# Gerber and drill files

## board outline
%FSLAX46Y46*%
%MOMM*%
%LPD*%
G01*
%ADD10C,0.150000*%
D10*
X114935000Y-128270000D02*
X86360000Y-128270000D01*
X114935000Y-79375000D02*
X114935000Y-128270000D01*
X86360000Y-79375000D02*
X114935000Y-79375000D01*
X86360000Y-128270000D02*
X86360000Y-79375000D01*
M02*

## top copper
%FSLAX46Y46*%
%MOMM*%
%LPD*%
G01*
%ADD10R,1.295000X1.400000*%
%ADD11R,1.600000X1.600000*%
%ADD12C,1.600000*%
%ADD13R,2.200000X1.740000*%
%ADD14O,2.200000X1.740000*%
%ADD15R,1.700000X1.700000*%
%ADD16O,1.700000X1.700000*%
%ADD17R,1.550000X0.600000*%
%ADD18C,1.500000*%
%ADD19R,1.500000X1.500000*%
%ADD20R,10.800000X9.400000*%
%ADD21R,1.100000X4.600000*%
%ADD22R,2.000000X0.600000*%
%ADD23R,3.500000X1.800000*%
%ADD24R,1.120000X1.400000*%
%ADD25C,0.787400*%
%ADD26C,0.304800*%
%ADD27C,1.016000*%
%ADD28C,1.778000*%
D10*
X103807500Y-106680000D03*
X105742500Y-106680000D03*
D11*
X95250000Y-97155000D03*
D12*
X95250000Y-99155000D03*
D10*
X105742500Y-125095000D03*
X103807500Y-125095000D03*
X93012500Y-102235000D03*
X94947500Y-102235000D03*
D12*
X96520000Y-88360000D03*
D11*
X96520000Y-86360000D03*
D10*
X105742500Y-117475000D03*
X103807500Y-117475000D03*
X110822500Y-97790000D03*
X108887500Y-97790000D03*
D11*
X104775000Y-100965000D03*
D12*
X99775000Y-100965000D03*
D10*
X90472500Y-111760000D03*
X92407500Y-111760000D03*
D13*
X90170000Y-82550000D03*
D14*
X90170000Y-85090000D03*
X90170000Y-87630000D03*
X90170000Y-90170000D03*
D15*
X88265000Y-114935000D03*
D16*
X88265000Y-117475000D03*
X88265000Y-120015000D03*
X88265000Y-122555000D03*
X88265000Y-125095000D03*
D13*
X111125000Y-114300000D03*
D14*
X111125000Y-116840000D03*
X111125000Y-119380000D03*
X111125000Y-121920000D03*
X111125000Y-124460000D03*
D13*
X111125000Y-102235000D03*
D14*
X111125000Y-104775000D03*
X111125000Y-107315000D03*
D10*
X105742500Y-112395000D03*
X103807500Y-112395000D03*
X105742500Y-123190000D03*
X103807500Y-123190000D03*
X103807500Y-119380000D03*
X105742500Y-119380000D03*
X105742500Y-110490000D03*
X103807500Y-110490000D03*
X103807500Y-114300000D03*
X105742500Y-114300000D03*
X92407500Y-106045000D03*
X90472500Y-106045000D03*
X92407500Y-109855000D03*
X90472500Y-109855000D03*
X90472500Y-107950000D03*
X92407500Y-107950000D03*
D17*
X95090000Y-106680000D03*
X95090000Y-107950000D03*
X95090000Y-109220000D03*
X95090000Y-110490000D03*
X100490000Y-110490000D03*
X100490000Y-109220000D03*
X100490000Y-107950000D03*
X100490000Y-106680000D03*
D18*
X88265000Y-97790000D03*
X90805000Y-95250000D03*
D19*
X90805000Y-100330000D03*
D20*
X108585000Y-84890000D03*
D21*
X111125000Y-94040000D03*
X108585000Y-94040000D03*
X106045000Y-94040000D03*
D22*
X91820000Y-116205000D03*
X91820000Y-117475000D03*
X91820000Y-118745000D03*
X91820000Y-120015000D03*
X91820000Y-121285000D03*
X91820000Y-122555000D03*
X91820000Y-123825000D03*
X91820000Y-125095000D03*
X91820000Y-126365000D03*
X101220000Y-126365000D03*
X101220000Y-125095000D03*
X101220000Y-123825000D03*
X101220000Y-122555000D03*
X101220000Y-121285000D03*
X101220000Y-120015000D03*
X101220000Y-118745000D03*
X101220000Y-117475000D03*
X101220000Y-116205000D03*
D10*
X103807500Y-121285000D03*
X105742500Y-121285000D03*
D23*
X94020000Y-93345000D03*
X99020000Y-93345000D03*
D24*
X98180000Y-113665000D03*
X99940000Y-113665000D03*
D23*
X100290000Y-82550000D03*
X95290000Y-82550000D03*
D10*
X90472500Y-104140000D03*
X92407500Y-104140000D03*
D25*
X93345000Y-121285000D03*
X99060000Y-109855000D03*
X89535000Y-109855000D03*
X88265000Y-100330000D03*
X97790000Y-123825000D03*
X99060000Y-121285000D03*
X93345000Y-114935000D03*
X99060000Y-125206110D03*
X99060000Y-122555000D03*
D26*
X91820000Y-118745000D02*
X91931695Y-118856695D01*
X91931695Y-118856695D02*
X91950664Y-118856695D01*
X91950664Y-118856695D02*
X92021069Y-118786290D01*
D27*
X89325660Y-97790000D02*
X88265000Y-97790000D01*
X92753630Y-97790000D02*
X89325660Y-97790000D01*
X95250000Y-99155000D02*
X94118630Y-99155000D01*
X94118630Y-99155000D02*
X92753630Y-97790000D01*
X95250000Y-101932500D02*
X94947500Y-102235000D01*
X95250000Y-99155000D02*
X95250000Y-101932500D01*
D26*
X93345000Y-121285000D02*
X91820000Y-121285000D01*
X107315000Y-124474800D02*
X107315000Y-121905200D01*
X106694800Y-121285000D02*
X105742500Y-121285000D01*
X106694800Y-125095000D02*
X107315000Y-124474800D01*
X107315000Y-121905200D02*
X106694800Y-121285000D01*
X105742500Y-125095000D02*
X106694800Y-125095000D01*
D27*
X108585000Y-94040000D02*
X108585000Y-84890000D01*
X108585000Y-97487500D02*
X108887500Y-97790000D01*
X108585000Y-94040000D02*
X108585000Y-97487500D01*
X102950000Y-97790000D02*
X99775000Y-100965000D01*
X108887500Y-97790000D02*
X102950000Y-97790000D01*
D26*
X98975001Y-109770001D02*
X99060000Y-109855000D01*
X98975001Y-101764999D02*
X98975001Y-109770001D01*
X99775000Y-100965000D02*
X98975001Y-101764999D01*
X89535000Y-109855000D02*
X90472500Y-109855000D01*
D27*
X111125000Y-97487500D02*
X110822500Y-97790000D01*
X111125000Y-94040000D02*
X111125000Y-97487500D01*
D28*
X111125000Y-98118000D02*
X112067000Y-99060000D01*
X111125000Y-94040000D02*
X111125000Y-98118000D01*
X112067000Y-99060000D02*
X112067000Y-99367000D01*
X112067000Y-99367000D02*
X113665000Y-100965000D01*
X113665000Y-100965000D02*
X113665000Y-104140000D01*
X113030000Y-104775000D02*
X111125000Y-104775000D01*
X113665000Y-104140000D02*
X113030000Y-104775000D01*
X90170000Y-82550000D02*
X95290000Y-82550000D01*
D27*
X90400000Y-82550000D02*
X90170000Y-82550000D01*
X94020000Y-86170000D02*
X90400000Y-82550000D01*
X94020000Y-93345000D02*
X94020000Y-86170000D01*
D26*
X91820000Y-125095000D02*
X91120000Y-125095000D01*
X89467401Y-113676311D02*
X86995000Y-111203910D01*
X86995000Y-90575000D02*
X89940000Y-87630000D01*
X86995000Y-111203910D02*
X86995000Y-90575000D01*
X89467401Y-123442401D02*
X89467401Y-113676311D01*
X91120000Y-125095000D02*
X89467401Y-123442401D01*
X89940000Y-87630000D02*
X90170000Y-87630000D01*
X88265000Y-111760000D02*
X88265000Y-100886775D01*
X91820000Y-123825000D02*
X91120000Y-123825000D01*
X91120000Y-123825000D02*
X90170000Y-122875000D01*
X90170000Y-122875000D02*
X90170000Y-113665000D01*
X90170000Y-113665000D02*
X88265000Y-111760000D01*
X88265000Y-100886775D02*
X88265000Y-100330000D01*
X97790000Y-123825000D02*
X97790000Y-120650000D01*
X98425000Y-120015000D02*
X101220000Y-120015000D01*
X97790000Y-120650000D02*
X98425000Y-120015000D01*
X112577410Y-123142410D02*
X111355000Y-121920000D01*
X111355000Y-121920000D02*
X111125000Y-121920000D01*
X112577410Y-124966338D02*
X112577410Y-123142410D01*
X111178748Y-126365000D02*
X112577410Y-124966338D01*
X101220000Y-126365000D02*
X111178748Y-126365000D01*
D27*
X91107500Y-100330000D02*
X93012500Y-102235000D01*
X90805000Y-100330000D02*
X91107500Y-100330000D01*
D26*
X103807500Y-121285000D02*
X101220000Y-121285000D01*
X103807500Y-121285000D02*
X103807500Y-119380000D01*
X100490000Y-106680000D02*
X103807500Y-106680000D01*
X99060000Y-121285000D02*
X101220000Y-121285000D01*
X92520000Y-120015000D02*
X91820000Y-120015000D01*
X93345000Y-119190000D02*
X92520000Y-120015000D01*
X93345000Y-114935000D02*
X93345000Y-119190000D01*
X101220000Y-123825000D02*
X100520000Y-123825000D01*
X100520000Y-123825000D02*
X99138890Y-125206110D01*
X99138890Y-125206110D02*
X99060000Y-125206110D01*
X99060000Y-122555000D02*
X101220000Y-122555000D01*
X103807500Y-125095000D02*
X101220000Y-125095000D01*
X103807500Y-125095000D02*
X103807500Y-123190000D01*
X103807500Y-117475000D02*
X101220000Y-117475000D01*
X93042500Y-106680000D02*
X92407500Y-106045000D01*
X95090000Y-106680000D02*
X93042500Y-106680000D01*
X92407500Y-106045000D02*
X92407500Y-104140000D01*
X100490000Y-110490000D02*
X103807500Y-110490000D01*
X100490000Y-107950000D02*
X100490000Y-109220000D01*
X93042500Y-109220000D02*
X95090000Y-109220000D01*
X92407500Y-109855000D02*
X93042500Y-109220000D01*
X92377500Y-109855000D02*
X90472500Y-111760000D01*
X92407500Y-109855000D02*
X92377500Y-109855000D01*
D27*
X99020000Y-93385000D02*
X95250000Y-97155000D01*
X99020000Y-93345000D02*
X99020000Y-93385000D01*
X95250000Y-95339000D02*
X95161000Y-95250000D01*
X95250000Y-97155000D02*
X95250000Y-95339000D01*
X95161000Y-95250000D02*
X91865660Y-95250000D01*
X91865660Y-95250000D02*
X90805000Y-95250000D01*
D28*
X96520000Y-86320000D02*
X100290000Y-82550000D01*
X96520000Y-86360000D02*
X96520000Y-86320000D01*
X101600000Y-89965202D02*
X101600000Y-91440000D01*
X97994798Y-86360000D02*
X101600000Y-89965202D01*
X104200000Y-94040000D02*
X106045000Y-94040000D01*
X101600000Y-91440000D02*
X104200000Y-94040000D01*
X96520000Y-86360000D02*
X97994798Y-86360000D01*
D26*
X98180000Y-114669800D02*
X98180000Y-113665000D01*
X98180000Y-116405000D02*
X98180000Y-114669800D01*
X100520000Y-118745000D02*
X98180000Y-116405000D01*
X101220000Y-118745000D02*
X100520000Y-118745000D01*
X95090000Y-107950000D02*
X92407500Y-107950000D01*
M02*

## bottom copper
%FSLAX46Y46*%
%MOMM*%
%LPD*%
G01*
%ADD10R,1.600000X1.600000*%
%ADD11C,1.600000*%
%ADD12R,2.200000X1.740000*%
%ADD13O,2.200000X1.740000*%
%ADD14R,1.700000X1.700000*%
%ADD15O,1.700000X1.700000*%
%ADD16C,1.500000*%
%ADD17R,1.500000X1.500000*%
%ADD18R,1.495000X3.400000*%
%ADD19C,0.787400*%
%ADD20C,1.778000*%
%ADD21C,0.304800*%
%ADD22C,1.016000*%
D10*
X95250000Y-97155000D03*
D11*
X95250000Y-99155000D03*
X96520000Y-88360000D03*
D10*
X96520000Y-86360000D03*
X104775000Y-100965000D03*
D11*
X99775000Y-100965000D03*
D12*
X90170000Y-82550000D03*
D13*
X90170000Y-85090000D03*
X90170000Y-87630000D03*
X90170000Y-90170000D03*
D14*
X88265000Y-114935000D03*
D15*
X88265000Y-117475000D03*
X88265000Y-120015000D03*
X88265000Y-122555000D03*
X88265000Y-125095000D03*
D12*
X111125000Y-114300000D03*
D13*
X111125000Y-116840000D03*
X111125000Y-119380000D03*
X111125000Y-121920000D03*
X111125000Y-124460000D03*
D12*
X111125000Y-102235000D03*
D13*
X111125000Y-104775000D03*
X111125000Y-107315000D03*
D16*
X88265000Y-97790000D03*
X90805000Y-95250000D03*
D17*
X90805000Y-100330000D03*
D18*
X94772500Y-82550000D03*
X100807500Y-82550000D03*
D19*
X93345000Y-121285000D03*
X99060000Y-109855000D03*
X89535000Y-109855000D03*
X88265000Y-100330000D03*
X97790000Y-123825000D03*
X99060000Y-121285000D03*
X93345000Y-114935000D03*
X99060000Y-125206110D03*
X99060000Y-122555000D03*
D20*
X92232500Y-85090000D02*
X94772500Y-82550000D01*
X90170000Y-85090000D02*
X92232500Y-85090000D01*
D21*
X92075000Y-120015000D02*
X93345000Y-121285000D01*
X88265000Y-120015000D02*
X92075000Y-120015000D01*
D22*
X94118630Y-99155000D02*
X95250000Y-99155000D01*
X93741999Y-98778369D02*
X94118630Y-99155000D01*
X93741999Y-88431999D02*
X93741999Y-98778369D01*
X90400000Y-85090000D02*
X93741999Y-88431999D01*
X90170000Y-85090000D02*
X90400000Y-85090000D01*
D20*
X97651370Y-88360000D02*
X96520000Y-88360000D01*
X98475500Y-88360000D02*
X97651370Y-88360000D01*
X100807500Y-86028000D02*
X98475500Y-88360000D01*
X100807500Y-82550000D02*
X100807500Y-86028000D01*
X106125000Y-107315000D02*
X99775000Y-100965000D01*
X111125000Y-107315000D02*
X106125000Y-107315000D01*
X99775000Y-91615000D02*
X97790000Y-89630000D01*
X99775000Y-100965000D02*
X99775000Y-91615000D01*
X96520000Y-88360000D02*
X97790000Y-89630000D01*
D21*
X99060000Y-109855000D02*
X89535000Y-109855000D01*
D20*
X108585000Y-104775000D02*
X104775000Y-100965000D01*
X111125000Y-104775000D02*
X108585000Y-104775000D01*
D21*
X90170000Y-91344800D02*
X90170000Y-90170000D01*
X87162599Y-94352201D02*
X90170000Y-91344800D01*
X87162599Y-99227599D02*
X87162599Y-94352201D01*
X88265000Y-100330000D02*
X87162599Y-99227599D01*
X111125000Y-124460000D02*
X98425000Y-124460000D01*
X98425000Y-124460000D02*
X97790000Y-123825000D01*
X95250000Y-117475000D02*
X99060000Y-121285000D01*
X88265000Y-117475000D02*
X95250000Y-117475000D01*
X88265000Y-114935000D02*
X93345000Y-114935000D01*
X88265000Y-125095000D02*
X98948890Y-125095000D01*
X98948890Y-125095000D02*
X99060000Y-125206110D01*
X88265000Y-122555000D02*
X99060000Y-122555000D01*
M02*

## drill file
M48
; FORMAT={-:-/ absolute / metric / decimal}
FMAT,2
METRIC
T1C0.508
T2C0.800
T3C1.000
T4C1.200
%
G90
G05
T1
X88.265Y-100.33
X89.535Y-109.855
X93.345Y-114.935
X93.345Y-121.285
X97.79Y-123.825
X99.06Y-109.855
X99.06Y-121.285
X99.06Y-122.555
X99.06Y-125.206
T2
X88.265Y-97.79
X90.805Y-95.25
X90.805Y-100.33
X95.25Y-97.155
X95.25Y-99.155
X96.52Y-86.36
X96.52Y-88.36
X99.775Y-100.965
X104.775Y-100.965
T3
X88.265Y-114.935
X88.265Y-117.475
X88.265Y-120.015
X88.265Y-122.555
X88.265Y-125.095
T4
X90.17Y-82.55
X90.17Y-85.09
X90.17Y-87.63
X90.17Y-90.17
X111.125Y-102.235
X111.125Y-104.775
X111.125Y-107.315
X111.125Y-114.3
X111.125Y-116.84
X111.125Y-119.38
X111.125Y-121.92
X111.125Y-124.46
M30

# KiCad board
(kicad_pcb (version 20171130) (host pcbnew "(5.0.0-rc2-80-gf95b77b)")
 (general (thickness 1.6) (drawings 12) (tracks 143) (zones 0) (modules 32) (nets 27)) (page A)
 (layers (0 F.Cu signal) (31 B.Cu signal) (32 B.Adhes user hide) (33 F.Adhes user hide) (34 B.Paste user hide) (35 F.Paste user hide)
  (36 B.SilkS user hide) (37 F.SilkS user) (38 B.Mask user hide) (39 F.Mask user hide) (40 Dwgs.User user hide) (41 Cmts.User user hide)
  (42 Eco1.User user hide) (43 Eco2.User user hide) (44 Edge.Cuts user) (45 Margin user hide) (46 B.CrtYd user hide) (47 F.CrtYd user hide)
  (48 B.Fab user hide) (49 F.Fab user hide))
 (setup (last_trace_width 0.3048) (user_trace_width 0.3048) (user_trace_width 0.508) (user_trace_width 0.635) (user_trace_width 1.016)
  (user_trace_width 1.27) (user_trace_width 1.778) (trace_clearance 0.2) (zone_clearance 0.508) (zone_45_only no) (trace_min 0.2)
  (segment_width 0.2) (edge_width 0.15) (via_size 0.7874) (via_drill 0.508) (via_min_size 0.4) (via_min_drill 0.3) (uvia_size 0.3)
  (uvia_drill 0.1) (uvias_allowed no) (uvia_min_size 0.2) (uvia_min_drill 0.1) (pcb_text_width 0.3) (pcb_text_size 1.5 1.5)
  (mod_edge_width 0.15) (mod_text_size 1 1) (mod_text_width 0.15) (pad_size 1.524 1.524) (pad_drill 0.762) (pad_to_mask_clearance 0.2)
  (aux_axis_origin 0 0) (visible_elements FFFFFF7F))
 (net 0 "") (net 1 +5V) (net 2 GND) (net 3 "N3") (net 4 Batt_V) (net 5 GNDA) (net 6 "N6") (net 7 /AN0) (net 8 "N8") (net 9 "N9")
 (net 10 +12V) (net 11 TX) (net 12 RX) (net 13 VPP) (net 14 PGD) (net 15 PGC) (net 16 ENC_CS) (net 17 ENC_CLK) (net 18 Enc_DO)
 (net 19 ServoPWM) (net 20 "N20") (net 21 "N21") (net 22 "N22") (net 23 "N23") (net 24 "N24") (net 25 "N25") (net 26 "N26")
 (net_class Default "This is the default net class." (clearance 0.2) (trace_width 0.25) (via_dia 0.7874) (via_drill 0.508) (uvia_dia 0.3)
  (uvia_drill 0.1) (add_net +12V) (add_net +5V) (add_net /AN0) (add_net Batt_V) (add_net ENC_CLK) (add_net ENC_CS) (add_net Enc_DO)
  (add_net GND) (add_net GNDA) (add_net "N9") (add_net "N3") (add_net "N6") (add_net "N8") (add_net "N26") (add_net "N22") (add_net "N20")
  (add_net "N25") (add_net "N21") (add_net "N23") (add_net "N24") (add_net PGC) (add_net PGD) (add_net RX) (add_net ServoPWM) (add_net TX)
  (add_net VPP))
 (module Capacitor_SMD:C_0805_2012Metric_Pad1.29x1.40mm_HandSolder (layer F.Cu) (at 104.775 106.68)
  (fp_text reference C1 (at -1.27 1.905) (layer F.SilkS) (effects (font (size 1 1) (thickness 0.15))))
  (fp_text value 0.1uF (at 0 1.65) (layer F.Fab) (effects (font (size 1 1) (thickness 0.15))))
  (pad 1 smd rect (at -0.9675 0) (size 1.295 1.4) (layers F.Cu F.Paste F.Mask) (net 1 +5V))
  (pad 2 smd rect (at 0.9675 0) (size 1.295 1.4) (layers F.Cu F.Paste F.Mask) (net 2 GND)))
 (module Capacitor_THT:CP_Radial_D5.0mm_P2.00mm (layer F.Cu) (at 95.25 97.155 270)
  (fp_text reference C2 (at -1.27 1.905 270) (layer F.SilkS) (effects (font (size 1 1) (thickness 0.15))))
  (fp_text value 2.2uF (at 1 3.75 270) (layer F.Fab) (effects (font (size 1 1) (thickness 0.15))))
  (pad 1 thru_hole rect (at 0 0 270) (size 1.6 1.6) (drill 0.8) (layers *.Cu *.Mask) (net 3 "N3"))
  (pad 2 thru_hole circle (at 2 0 270) (size 1.6 1.6) (drill 0.8) (layers *.Cu *.Mask) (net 2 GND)))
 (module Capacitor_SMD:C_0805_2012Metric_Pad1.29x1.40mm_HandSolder (layer F.Cu) (at 104.775 125.095)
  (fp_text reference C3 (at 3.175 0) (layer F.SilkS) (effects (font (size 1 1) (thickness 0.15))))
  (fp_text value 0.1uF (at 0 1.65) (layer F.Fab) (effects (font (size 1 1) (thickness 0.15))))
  (pad 2 smd rect (at 0.9675 0) (size 1.295 1.4) (layers F.Cu F.Paste F.Mask) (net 2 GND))
  (pad 1 smd rect (at -0.9675 0) (size 1.295 1.4) (layers F.Cu F.Paste F.Mask) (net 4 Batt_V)))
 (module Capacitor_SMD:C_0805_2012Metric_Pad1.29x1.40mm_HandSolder (layer F.Cu) (at 93.98 102.235)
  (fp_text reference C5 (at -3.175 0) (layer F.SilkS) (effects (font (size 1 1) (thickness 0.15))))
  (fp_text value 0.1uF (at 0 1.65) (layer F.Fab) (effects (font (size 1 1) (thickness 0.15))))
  (pad 1 smd rect (at -0.9675 0) (size 1.295 1.4) (layers F.Cu F.Paste F.Mask) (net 1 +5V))
  (pad 2 smd rect (at 0.9675 0) (size 1.295 1.4) (layers F.Cu F.Paste F.Mask) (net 2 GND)))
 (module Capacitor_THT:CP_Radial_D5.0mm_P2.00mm (layer F.Cu) (at 96.52 86.36 270)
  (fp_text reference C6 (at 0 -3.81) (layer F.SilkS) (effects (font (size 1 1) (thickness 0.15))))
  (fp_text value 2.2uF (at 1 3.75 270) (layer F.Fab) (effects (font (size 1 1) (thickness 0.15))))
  (pad 2 thru_hole circle (at 2 0 270) (size 1.6 1.6) (drill 0.8) (layers *.Cu *.Mask) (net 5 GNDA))
  (pad 1 thru_hole rect (at 0 0 270) (size 1.6 1.6) (drill 0.8) (layers *.Cu *.Mask) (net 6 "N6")))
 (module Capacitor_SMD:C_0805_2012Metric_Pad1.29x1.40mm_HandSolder (layer F.Cu) (at 104.775 117.475)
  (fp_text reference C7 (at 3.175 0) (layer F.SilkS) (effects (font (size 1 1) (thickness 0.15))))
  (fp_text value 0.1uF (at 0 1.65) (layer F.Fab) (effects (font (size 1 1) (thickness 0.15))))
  (pad 2 smd rect (at 0.9675 0) (size 1.295 1.4) (layers F.Cu F.Paste F.Mask) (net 2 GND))
  (pad 1 smd rect (at -0.9675 0) (size 1.295 1.4) (layers F.Cu F.Paste F.Mask) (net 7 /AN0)))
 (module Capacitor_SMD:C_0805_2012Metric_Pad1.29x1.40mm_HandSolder (layer F.Cu) (at 109.855 97.79 180)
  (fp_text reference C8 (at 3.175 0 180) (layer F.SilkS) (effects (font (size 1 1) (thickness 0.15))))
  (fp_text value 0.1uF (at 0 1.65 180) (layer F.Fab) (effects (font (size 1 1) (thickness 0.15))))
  (pad 1 smd rect (at -0.9675 0 180) (size 1.295 1.4) (layers F.Cu F.Paste F.Mask) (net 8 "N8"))
  (pad 2 smd rect (at 0.9675 0 180) (size 1.295 1.4) (layers F.Cu F.Paste F.Mask) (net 5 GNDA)))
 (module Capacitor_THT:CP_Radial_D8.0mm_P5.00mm (layer F.Cu) (at 104.775 100.965 180)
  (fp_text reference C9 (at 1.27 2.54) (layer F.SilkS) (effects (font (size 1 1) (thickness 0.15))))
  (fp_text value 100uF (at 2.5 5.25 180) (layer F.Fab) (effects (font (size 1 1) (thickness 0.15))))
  (pad 1 thru_hole rect (at 0 0 180) (size 1.6 1.6) (drill 0.8) (layers *.Cu *.Mask) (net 8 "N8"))
  (pad 2 thru_hole circle (at 5 0 180) (size 1.6 1.6) (drill 0.8) (layers *.Cu *.Mask) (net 5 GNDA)))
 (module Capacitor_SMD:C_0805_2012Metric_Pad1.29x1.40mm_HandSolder (layer F.Cu) (at 91.44 111.76)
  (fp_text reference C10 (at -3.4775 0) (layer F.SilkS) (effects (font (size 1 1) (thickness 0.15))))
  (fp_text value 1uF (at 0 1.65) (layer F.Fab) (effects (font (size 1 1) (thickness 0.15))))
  (pad 1 smd rect (at -0.9675 0) (size 1.295 1.4) (layers F.Cu F.Paste F.Mask) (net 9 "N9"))
  (pad 2 smd rect (at 0.9675 0) (size 1.295 1.4) (layers F.Cu F.Paste F.Mask) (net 2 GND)))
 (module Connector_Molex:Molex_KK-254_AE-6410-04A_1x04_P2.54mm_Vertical (layer F.Cu) (at 90.17 82.55 270)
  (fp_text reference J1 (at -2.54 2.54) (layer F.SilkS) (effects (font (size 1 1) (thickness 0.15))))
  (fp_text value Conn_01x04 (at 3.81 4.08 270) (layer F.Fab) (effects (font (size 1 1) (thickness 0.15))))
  (pad 1 thru_hole rect (at 0 0 270) (size 1.74 2.2) (drill 1.2) (layers *.Cu *.Mask) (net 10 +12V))
  (pad 2 thru_hole oval (at 2.54 0 270) (size 1.74 2.2) (drill 1.2) (layers *.Cu *.Mask) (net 2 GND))
  (pad 3 thru_hole oval (at 5.08 0 270) (size 1.74 2.2) (drill 1.2) (layers *.Cu *.Mask) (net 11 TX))
  (pad 4 thru_hole oval (at 7.62 0 270) (size 1.74 2.2) (drill 1.2) (layers *.Cu *.Mask) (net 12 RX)))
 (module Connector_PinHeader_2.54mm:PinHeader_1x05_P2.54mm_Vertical (layer F.Cu) (at 88.265 114.935)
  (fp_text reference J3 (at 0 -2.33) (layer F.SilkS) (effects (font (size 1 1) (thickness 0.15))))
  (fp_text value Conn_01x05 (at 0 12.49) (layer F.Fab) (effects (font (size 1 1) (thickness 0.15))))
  (pad 1 thru_hole rect (at 0 0) (size 1.7 1.7) (drill 1) (layers *.Cu *.Mask) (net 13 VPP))
  (pad 2 thru_hole oval (at 0 2.54) (size 1.7 1.7) (drill 1) (layers *.Cu *.Mask) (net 1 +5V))
  (pad 3 thru_hole oval (at 0 5.08) (size 1.7 1.7) (drill 1) (layers *.Cu *.Mask) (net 2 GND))
  (pad 4 thru_hole oval (at 0 7.62) (size 1.7 1.7) (drill 1) (layers *.Cu *.Mask) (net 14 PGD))
  (pad 5 thru_hole oval (at 0 10.16) (size 1.7 1.7) (drill 1) (layers *.Cu *.Mask) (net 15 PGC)))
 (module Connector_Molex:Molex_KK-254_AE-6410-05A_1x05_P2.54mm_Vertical (layer F.Cu) (at 111.125 114.3 270)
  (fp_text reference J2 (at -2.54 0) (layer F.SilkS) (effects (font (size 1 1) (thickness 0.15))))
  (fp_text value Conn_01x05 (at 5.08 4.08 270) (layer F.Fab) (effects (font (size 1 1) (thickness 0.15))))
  (pad 1 thru_hole rect (at 0 0 270) (size 1.74 2.2) (drill 1.2) (layers *.Cu *.Mask) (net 1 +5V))
  (pad 2 thru_hole oval (at 2.54 0 270) (size 1.74 2.2) (drill 1.2) (layers *.Cu *.Mask) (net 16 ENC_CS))
  (pad 3 thru_hole oval (at 5.08 0 270) (size 1.74 2.2) (drill 1.2) (layers *.Cu *.Mask) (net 2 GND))
  (pad 4 thru_hole oval (at 7.62 0 270) (size 1.74 2.2) (drill 1.2) (layers *.Cu *.Mask) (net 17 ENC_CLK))
  (pad 5 thru_hole oval (at 10.16 0 270) (size 1.74 2.2) (drill 1.2) (layers *.Cu *.Mask) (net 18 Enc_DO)))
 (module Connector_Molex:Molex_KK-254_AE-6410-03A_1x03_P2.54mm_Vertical (layer F.Cu) (at 111.125 102.235 270)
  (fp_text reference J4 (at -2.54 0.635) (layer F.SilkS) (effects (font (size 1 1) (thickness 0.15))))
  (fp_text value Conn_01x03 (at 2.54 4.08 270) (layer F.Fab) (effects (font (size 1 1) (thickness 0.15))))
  (pad 1 thru_hole rect (at 0 0 270) (size 1.74 2.2) (drill 1.2) (layers *.Cu *.Mask) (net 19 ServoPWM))
  (pad 2 thru_hole oval (at 2.54 0 270) (size 1.74 2.2) (drill 1.2) (layers *.Cu *.Mask) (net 8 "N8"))
  (pad 3 thru_hole oval (at 5.08 0 270) (size 1.74 2.2) (drill 1.2) (layers *.Cu *.Mask) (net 5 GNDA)))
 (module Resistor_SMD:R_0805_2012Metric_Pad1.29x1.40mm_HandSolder (layer F.Cu) (at 104.775 112.395)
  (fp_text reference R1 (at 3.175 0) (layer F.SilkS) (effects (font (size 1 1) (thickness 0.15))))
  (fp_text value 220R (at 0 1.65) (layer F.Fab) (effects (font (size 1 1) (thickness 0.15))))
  (pad 2 smd rect (at 0.9675 0) (size 1.295 1.4) (layers F.Cu F.Paste F.Mask) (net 19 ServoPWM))
  (pad 1 smd rect (at -0.9675 0) (size 1.295 1.4) (layers F.Cu F.Paste F.Mask) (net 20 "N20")))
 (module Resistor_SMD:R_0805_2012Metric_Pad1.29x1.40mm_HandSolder (layer F.Cu) (at 104.775 123.19 180)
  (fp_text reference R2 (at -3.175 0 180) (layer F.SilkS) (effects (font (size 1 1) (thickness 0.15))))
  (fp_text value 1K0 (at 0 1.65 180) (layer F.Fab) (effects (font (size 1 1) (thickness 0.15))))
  (pad 1 smd rect (at -0.9675 0 180) (size 1.295 1.4) (layers F.Cu F.Paste F.Mask) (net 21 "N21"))
  (pad 2 smd rect (at 0.9675 0 180) (size 1.295 1.4) (layers F.Cu F.Paste F.Mask) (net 4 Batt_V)))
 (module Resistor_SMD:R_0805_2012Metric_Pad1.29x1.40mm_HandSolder (layer F.Cu) (at 104.775 119.38 180)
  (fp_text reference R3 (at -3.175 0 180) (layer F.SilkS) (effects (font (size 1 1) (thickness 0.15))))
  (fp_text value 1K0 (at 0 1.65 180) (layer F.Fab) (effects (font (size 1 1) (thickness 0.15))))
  (pad 2 smd rect (at 0.9675 0 180) (size 1.295 1.4) (layers F.Cu F.Paste F.Mask) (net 1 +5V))
  (pad 1 smd rect (at -0.9675 0 180) (size 1.295 1.4) (layers F.Cu F.Paste F.Mask) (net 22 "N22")))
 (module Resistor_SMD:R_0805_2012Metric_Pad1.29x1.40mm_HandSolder (layer F.Cu) (at 104.775 110.49 180)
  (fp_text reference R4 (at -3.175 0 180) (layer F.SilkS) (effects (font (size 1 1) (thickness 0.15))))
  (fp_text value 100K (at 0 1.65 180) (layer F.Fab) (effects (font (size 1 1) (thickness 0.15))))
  (pad 1 smd rect (at -0.9675 0 180) (size 1.295 1.4) (layers F.Cu F.Paste F.Mask) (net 10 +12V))
  (pad 2 smd rect (at 0.9675 0 180) (size 1.295 1.4) (layers F.Cu F.Paste F.Mask) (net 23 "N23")))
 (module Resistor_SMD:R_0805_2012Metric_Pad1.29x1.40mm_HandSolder (layer F.Cu) (at 104.775 114.3 180)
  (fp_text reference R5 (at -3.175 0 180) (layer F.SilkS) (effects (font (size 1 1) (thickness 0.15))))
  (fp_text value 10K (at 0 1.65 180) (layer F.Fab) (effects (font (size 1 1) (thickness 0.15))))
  (pad 2 smd rect (at 0.9675 0 180) (size 1.295 1.4) (layers F.Cu F.Paste F.Mask) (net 23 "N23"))
  (pad 1 smd rect (at -0.9675 0 180) (size 1.295 1.4) (layers F.Cu F.Paste F.Mask) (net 2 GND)))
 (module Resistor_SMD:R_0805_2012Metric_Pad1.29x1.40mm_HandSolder (layer F.Cu) (at 91.44 106.045 180)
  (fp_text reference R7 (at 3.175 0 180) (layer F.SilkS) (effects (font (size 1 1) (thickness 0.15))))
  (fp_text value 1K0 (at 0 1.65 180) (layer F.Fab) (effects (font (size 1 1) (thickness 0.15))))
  (pad 1 smd rect (at -0.9675 0 180) (size 1.295 1.4) (layers F.Cu F.Paste F.Mask) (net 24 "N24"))
  (pad 2 smd rect (at 0.9675 0 180) (size 1.295 1.4) (layers F.Cu F.Paste F.Mask) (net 7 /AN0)))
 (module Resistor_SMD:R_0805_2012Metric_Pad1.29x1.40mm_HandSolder (layer F.Cu) (at 91.44 109.855)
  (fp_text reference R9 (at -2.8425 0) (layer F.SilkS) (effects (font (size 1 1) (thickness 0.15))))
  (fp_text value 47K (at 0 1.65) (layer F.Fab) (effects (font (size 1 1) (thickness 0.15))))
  (pad 2 smd rect (at 0.9675 0) (size 1.295 1.4) (layers F.Cu F.Paste F.Mask) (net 9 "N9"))
  (pad 1 smd rect (at -0.9675 0) (size 1.295 1.4) (layers F.Cu F.Paste F.Mask) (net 5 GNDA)))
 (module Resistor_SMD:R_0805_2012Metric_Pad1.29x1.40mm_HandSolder (layer F.Cu) (at 91.44 107.95)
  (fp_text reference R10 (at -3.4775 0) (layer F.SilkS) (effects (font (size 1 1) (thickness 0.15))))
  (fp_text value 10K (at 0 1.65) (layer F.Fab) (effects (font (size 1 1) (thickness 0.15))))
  (pad 1 smd rect (at -0.9675 0) (size 1.295 1.4) (layers F.Cu F.Paste F.Mask) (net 2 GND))
  (pad 2 smd rect (at 0.9675 0) (size 1.295 1.4) (layers F.Cu F.Paste F.Mask) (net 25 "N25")))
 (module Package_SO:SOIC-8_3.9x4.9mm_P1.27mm (layer F.Cu) (at 97.79 108.585)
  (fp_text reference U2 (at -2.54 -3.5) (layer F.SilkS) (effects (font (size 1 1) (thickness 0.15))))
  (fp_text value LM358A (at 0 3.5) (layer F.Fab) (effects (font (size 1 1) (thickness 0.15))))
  (pad 1 smd rect (at -2.7 -1.905) (size 1.55 0.6) (layers F.Cu F.Paste F.Mask) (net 24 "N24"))
  (pad 2 smd rect (at -2.7 -0.635) (size 1.55 0.6) (layers F.Cu F.Paste F.Mask) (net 25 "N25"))
  (pad 3 smd rect (at -2.7 0.635) (size 1.55 0.6) (layers F.Cu F.Paste F.Mask) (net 9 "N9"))
  (pad 4 smd rect (at -2.7 1.905) (size 1.55 0.6) (layers F.Cu F.Paste F.Mask) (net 2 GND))
  (pad 5 smd rect (at 2.7 1.905) (size 1.55 0.6) (layers F.Cu F.Paste F.Mask) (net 23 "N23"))
  (pad 6 smd rect (at 2.7 0.635) (size 1.55 0.6) (layers F.Cu F.Paste F.Mask) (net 21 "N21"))
  (pad 7 smd rect (at 2.7 -0.635) (size 1.55 0.6) (layers F.Cu F.Paste F.Mask) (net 21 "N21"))
  (pad 8 smd rect (at 2.7 -1.905) (size 1.55 0.6) (layers F.Cu F.Paste F.Mask) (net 1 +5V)))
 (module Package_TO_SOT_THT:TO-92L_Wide (layer F.Cu) (at 90.805 100.33 90)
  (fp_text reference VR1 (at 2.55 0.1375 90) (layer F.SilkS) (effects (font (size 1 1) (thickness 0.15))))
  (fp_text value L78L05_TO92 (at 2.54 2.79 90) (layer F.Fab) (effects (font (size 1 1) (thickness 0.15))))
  (pad 2 thru_hole circle (at 2.54 -2.54 180) (size 1.5 1.5) (drill 0.8) (layers *.Cu *.Mask) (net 2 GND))
  (pad 3 thru_hole circle (at 5.08 0 180) (size 1.5 1.5) (drill 0.8) (layers *.Cu *.Mask) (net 3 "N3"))
  (pad 1 thru_hole rect (at 0 0 180) (size 1.5 1.5) (drill 0.8) (layers *.Cu *.Mask) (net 1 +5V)))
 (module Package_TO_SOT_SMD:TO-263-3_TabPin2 (layer F.Cu) (at 108.585 88.265 90)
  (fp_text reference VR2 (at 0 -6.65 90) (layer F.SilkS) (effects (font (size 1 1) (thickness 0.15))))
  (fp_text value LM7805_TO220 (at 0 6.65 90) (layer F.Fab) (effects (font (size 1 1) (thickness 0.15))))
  (pad "" smd rect (at 0.95 2.775 90) (size 4.55 5.25) (layers F.Paste))
  (pad "" smd rect (at 5.8 -2.775 90) (size 4.55 5.25) (layers F.Paste))
  (pad "" smd rect (at 0.95 -2.775 90) (size 4.55 5.25) (layers F.Paste))
  (pad "" smd rect (at 5.8 2.775 90) (size 4.55 5.25) (layers F.Paste))
  (pad 2 smd rect (at 3.375 0 90) (size 9.4 10.8) (layers F.Cu F.Mask) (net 5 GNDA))
  (pad 3 smd rect (at -5.775 2.54 90) (size 4.6 1.1) (layers F.Cu F.Paste F.Mask) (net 8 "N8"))
  (pad 2 smd rect (at -5.775 0 90) (size 4.6 1.1) (layers F.Cu F.Paste F.Mask) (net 5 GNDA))
  (pad 1 smd rect (at -5.775 -2.54 90) (size 4.6 1.1) (layers F.Cu F.Paste F.Mask) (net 6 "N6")))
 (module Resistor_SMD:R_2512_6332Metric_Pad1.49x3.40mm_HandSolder (layer B.Cu) (at 97.79 82.55)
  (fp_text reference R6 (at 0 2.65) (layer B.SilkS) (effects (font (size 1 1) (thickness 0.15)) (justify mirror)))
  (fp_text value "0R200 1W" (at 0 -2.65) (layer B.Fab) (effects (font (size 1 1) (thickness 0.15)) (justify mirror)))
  (pad 1 smd rect (at -3.0175 0) (size 1.495 3.4) (layers B.Cu B.Paste B.Mask) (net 2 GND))
  (pad 2 smd rect (at 3.0175 0) (size 1.495 3.4) (layers B.Cu B.Paste B.Mask) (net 5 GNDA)))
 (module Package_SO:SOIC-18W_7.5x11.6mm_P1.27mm (layer F.Cu) (at 96.52 121.285)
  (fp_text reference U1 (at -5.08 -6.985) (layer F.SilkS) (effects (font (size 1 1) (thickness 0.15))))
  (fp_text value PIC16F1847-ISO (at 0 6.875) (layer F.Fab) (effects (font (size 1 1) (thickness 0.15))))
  (pad 1 smd rect (at -4.7 -5.08) (size 2 0.6) (layers F.Cu F.Paste F.Mask))
  (pad 2 smd rect (at -4.7 -3.81) (size 2 0.6) (layers F.Cu F.Paste F.Mask))
  (pad 3 smd rect (at -4.7 -2.54) (size 2 0.6) (layers F.Cu F.Paste F.Mask))
  (pad 4 smd rect (at -4.7 -1.27) (size 2 0.6) (layers F.Cu F.Paste F.Mask) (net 13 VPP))
  (pad 5 smd rect (at -4.7 0) (size 2 0.6) (layers F.Cu F.Paste F.Mask) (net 2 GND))
  (pad 6 smd rect (at -4.7 1.27) (size 2 0.6) (layers F.Cu F.Paste F.Mask) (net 16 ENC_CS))
  (pad 7 smd rect (at -4.7 2.54) (size 2 0.6) (layers F.Cu F.Paste F.Mask) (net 12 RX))
  (pad 8 smd rect (at -4.7 3.81) (size 2 0.6) (layers F.Cu F.Paste F.Mask) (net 11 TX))
  (pad 9 smd rect (at -4.7 5.08) (size 2 0.6) (layers F.Cu F.Paste F.Mask) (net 20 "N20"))
  (pad 10 smd rect (at 4.7 5.08) (size 2 0.6) (layers F.Cu F.Paste F.Mask) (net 17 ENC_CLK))
  (pad 11 smd rect (at 4.7 3.81) (size 2 0.6) (layers F.Cu F.Paste F.Mask) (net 4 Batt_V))
  (pad 12 smd rect (at 4.7 2.54) (size 2 0.6) (layers F.Cu F.Paste F.Mask) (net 15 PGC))
  (pad 13 smd rect (at 4.7 1.27) (size 2 0.6) (layers F.Cu F.Paste F.Mask) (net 14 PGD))
  (pad 14 smd rect (at 4.7 0) (size 2 0.6) (layers F.Cu F.Paste F.Mask) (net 1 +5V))
  (pad 15 smd rect (at 4.7 -1.27) (size 2 0.6) (layers F.Cu F.Paste F.Mask) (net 18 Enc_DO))
  (pad 16 smd rect (at 4.7 -2.54) (size 2 0.6) (layers F.Cu F.Paste F.Mask) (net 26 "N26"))
  (pad 17 smd rect (at 4.7 -3.81) (size 2 0.6) (layers F.Cu F.Paste F.Mask) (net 7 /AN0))
  (pad 18 smd rect (at 4.7 -5.08) (size 2 0.6) (layers F.Cu F.Paste F.Mask)))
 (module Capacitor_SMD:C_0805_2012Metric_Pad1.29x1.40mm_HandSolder (layer F.Cu) (at 104.775 121.285)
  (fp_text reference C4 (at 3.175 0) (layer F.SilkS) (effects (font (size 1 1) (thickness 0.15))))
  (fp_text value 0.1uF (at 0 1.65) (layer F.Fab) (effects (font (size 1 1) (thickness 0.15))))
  (pad 1 smd rect (at -0.9675 0) (size 1.295 1.4) (layers F.Cu F.Paste F.Mask) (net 1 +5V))
  (pad 2 smd rect (at 0.9675 0) (size 1.295 1.4) (layers F.Cu F.Paste F.Mask) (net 2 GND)))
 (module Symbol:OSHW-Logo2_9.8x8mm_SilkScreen (layer B.Cu) (at 94.615 111.76 180)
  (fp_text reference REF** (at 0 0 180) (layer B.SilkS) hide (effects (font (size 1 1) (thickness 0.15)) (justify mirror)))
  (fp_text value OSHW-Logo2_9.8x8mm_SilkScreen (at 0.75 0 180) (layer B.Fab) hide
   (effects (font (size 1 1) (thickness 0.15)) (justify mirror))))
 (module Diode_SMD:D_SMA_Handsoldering (layer F.Cu) (at 96.52 93.345 180)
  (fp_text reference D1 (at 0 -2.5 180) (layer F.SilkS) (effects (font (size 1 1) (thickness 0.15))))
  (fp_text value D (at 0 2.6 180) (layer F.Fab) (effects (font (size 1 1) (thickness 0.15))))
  (pad 2 smd rect (at 2.5 0 180) (size 3.5 1.8) (layers F.Cu F.Paste F.Mask) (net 10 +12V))
  (pad 1 smd rect (at -2.5 0 180) (size 3.5 1.8) (layers F.Cu F.Paste F.Mask) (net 3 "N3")))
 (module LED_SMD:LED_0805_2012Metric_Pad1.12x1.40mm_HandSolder (layer F.Cu) (at 99.06 113.665)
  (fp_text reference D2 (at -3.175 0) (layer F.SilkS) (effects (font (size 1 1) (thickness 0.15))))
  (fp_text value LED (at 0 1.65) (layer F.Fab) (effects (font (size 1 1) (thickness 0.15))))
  (pad 1 smd rect (at -0.88 0) (size 1.12 1.4) (layers F.Cu F.Paste F.Mask) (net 26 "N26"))
  (pad 2 smd rect (at 0.88 0) (size 1.12 1.4) (layers F.Cu F.Paste F.Mask) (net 22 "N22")))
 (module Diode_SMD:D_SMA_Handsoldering (layer F.Cu) (at 97.79 82.55 180)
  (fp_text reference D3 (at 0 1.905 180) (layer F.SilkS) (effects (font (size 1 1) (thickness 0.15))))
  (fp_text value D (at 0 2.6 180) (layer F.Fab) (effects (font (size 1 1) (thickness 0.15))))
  (pad 1 smd rect (at -2.5 0 180) (size 3.5 1.8) (layers F.Cu F.Paste F.Mask) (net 6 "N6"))
  (pad 2 smd rect (at 2.5 0 180) (size 3.5 1.8) (layers F.Cu F.Paste F.Mask) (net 10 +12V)))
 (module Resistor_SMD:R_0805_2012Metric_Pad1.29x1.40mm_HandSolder (layer F.Cu) (at 91.44 104.14)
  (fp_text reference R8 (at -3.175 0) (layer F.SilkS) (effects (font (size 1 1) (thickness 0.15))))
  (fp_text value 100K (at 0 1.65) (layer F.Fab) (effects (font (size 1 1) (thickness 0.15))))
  (pad 1 smd rect (at -0.9675 0) (size 1.295 1.4) (layers F.Cu F.Paste F.Mask) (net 25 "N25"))
  (pad 2 smd rect (at 0.9675 0) (size 1.295 1.4) (layers F.Cu F.Paste F.Mask) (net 24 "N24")))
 (gr_line (start 114.935 128.27) (end 86.36 128.27) (layer Edge.Cuts) (width 0.15))
 (gr_line (start 114.935 79.375) (end 114.935 128.27) (layer Edge.Cuts) (width 0.15))
 (gr_line (start 86.36 79.375) (end 114.935 79.375) (layer Edge.Cuts) (width 0.15))
 (gr_line (start 86.36 128.27) (end 86.36 79.375) (layer Edge.Cuts) (width 0.15))
 (segment (start 91.82 118.745) (end 91.931695 118.856695) (width 0.3048) (layer F.Cu) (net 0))
 (segment (start 91.931695 118.856695) (end 91.950664 118.856695) (width 0.3048) (layer F.Cu) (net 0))
 (segment (start 91.950664 118.856695) (end 92.021069 118.78629) (width 0.3048) (layer F.Cu) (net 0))
 (segment (start 92.2325 85.09) (end 94.7725 82.55) (width 1.778) (layer B.Cu) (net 2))
 (segment (start 90.17 85.09) (end 92.2325 85.09) (width 1.778) (layer B.Cu) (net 2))
 (segment (start 89.32566 97.79) (end 88.265 97.79) (width 1.016) (layer F.Cu) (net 2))
 (segment (start 92.75363 97.79) (end 89.32566 97.79) (width 1.016) (layer F.Cu) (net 2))
 (segment (start 95.25 99.155) (end 94.11863 99.155) (width 1.016) (layer F.Cu) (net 2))
 (segment (start 94.11863 99.155) (end 92.75363 97.79) (width 1.016) (layer F.Cu) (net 2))
 (segment (start 95.25 101.9325) (end 94.9475 102.235) (width 1.016) (layer F.Cu) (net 2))
 (segment (start 95.25 99.155) (end 95.25 101.9325) (width 1.016) (layer F.Cu) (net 2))
 (via (at 93.345 121.285) (size 0.7874) (drill 0.508) (layers F.Cu B.Cu) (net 2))
 (segment (start 92.075 120.015) (end 93.345 121.285) (width 0.3048) (layer B.Cu) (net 2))
 (segment (start 88.265 120.015) (end 92.075 120.015) (width 0.3048) (layer B.Cu) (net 2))
 (segment (start 93.345 121.285) (end 91.82 121.285) (width 0.3048) (layer F.Cu) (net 2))
 (segment (start 107.315 124.4748) (end 107.315 121.9052) (width 0.3048) (layer F.Cu) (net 2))
 (segment (start 106.6948 121.285) (end 105.7425 121.285) (width 0.3048) (layer F.Cu) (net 2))
 (segment (start 106.6948 125.095) (end 107.315 124.4748) (width 0.3048) (layer F.Cu) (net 2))
 (segment (start 107.315 121.9052) (end 106.6948 121.285) (width 0.3048) (layer F.Cu) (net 2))
 (segment (start 105.7425 125.095) (end 106.6948 125.095) (width 0.3048) (layer F.Cu) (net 2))
 (segment (start 94.11863 99.155) (end 95.25 99.155) (width 1.016) (layer B.Cu) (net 2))
 (segment (start 93.741999 98.778369) (end 94.11863 99.155) (width 1.016) (layer B.Cu) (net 2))
 (segment (start 93.741999 88.431999) (end 93.741999 98.778369) (width 1.016) (layer B.Cu) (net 2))
 (segment (start 90.4 85.09) (end 93.741999 88.431999) (width 1.016) (layer B.Cu) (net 2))
 (segment (start 90.17 85.09) (end 90.4 85.09) (width 1.016) (layer B.Cu) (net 2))
 (segment (start 108.585 94.04) (end 108.585 84.89) (width 1.016) (layer F.Cu) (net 5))
 (segment (start 97.65137 88.36) (end 96.52 88.36) (width 1.778) (layer B.Cu) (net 5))
 (segment (start 98.4755 88.36) (end 97.65137 88.36) (width 1.778) (layer B.Cu) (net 5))
 (segment (start 100.8075 86.028) (end 98.4755 88.36) (width 1.778) (layer B.Cu) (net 5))
 (segment (start 100.8075 82.55) (end 100.8075 86.028) (width 1.778) (layer B.Cu) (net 5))
 (segment (start 108.585 97.4875) (end 108.8875 97.79) (width 1.016) (layer F.Cu) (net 5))
 (segment (start 108.585 94.04) (end 108.585 97.4875) (width 1.016) (layer F.Cu) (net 5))
 (segment (start 106.125 107.315) (end 99.775 100.965) (width 1.778) (layer B.Cu) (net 5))
 (segment (start 111.125 107.315) (end 106.125 107.315) (width 1.778) (layer B.Cu) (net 5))
 (segment (start 99.775 91.615) (end 97.79 89.63) (width 1.778) (layer B.Cu) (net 5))
 (segment (start 99.775 100.965) (end 99.775 91.615) (width 1.778) (layer B.Cu) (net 5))
 (segment (start 96.52 88.36) (end 97.79 89.63) (width 1.778) (layer B.Cu) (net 5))
 (segment (start 102.95 97.79) (end 99.775 100.965) (width 1.016) (layer F.Cu) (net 5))
 (segment (start 108.8875 97.79) (end 102.95 97.79) (width 1.016) (layer F.Cu) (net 5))
 (via (at 99.06 109.855) (size 0.7874) (drill 0.508) (layers F.Cu B.Cu) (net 5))
 (segment (start 98.975001 109.770001) (end 99.06 109.855) (width 0.3048) (layer F.Cu) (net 5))
 (segment (start 98.975001 101.764999) (end 98.975001 109.770001) (width 0.3048) (layer F.Cu) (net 5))
 (segment (start 99.775 100.965) (end 98.975001 101.764999) (width 0.3048) (layer F.Cu) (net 5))
 (via (at 89.535 109.855) (size 0.7874) (drill 0.508) (layers F.Cu B.Cu) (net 5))
 (segment (start 99.06 109.855) (end 89.535 109.855) (width 0.3048) (layer B.Cu) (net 5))
 (segment (start 89.535 109.855) (end 90.4725 109.855) (width 0.3048) (layer F.Cu) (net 5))
 (segment (start 111.125 97.4875) (end 110.8225 97.79) (width 1.016) (layer F.Cu) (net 8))
 (segment (start 111.125 94.04) (end 111.125 97.4875) (width 1.016) (layer F.Cu) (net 8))
 (segment (start 111.125 98.118) (end 112.067 99.06) (width 1.778) (layer F.Cu) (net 8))
 (segment (start 111.125 94.04) (end 111.125 98.118) (width 1.778) (layer F.Cu) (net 8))
 (segment (start 112.067 99.06) (end 112.067 99.367) (width 1.778) (layer F.Cu) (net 8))
 (segment (start 112.067 99.367) (end 113.665 100.965) (width 1.778) (layer F.Cu) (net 8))
 (segment (start 113.665 100.965) (end 113.665 104.14) (width 1.778) (layer F.Cu) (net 8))
 (segment (start 113.03 104.775) (end 111.125 104.775) (width 1.778) (layer F.Cu) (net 8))
 (segment (start 113.665 104.14) (end 113.03 104.775) (width 1.778) (layer F.Cu) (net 8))
 (segment (start 108.585 104.775) (end 104.775 100.965) (width 1.778) (layer B.Cu) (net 8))
 (segment (start 111.125 104.775) (end 108.585 104.775) (width 1.778) (layer B.Cu) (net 8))
 (segment (start 90.17 82.55) (end 95.29 82.55) (width 1.778) (layer F.Cu) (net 10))
 (segment (start 90.4 82.55) (end 90.17 82.55) (width 1.016) (layer F.Cu) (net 10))
 (segment (start 94.02 86.17) (end 90.4 82.55) (width 1.016) (layer F.Cu) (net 10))
 (segment (start 94.02 93.345) (end 94.02 86.17) (width 1.016) (layer F.Cu) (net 10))
 (segment (start 91.82 125.095) (end 91.12 125.095) (width 0.3048) (layer F.Cu) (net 11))
 (segment (start 89.467401 113.676311) (end 86.995 111.20391) (width 0.3048) (layer F.Cu) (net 11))
 (segment (start 86.995 90.575) (end 89.94 87.63) (width 0.3048) (layer F.Cu) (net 11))
 (segment (start 86.995 111.20391) (end 86.995 90.575) (width 0.3048) (layer F.Cu) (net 11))
 (segment (start 89.467401 123.442401) (end 89.467401 113.676311) (width 0.3048) (layer F.Cu) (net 11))
 (segment (start 91.12 125.095) (end 89.467401 123.442401) (width 0.3048) (layer F.Cu) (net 11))
 (segment (start 89.94 87.63) (end 90.17 87.63) (width 0.3048) (layer F.Cu) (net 11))
 (via (at 88.265 100.33) (size 0.7874) (drill 0.508) (layers F.Cu B.Cu) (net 12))
 (segment (start 90.17 91.3448) (end 90.17 90.17) (width 0.3048) (layer B.Cu) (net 12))
 (segment (start 87.162599 94.352201) (end 90.17 91.3448) (width 0.3048) (layer B.Cu) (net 12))
 (segment (start 87.162599 99.227599) (end 87.162599 94.352201) (width 0.3048) (layer B.Cu) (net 12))
 (segment (start 88.265 100.33) (end 87.162599 99.227599) (width 0.3048) (layer B.Cu) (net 12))
 (segment (start 88.265 111.76) (end 88.265 100.886775) (width 0.3048) (layer F.Cu) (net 12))
 (segment (start 91.82 123.825) (end 91.12 123.825) (width 0.3048) (layer F.Cu) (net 12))
 (segment (start 91.12 123.825) (end 90.17 122.875) (width 0.3048) (layer F.Cu) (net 12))
 (segment (start 90.17 122.875) (end 90.17 113.665) (width 0.3048) (layer F.Cu) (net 12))
 (segment (start 90.17 113.665) (end 88.265 111.76) (width 0.3048) (layer F.Cu) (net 12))
 (segment (start 88.265 100.886775) (end 88.265 100.33) (width 0.3048) (layer F.Cu) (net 12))
 (via (at 97.79 123.825) (size 0.7874) (drill 0.508) (layers F.Cu B.Cu) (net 18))
 (segment (start 111.125 124.46) (end 98.425 124.46) (width 0.3048) (layer B.Cu) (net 18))
 (segment (start 98.425 124.46) (end 97.79 123.825) (width 0.3048) (layer B.Cu) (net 18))
 (segment (start 97.79 123.825) (end 97.79 120.65) (width 0.3048) (layer F.Cu) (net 18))
 (segment (start 98.425 120.015) (end 101.22 120.015) (width 0.3048) (layer F.Cu) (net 18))
 (segment (start 97.79 120.65) (end 98.425 120.015) (width 0.3048) (layer F.Cu) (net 18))
 (segment (start 112.57741 123.14241) (end 111.355 121.92) (width 0.3048) (layer F.Cu) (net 17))
 (segment (start 111.355 121.92) (end 111.125 121.92) (width 0.3048) (layer F.Cu) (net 17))
 (segment (start 112.57741 124.966338) (end 112.57741 123.14241) (width 0.3048) (layer F.Cu) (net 17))
 (segment (start 111.178748 126.365) (end 112.57741 124.966338) (width 0.3048) (layer F.Cu) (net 17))
 (segment (start 101.22 126.365) (end 111.178748 126.365) (width 0.3048) (layer F.Cu) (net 17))
 (segment (start 91.1075 100.33) (end 93.0125 102.235) (width 1.016) (layer F.Cu) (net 1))
 (segment (start 90.805 100.33) (end 91.1075 100.33) (width 1.016) (layer F.Cu) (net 1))
 (segment (start 103.8075 121.285) (end 101.22 121.285) (width 0.3048) (layer F.Cu) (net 1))
 (segment (start 103.8075 121.285) (end 103.8075 119.38) (width 0.3048) (layer F.Cu) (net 1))
 (segment (start 100.49 106.68) (end 103.8075 106.68) (width 0.3048) (layer F.Cu) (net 1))
 (via (at 99.06 121.285) (size 0.7874) (drill 0.508) (layers F.Cu B.Cu) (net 1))
 (segment (start 95.25 117.475) (end 99.06 121.285) (width 0.3048) (layer B.Cu) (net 1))
 (segment (start 88.265 117.475) (end 95.25 117.475) (width 0.3048) (layer B.Cu) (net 1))
 (segment (start 99.06 121.285) (end 101.22 121.285) (width 0.3048) (layer F.Cu) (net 1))
 (via (at 93.345 114.935) (size 0.7874) (drill 0.508) (layers F.Cu B.Cu) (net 13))
 (segment (start 88.265 114.935) (end 93.345 114.935) (width 0.3048) (layer B.Cu) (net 13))
 (segment (start 92.52 120.015) (end 91.82 120.015) (width 0.3048) (layer F.Cu) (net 13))
 (segment (start 93.345 119.19) (end 92.52 120.015) (width 0.3048) (layer F.Cu) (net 13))
 (segment (start 93.345 114.935) (end 93.345 119.19) (width 0.3048) (layer F.Cu) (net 13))
 (segment (start 101.22 123.825) (end 100.52 123.825) (width 0.3048) (layer F.Cu) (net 15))
 (segment (start 88.265 125.095) (end 98.94889 125.095) (width 0.3048) (layer B.Cu) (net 15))
 (via (at 99.06 125.20611) (size 0.7874) (drill 0.508) (layers F.Cu B.Cu) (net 15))
 (segment (start 98.94889 125.095) (end 99.06 125.20611) (width 0.3048) (layer B.Cu) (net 15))
 (segment (start 100.52 123.825) (end 99.13889 125.20611) (width 0.3048) (layer F.Cu) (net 15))
 (segment (start 99.13889 125.20611) (end 99.06 125.20611) (width 0.3048) (layer F.Cu) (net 15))
 (via (at 99.06 122.555) (size 0.7874) (drill 0.508) (layers F.Cu B.Cu) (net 14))
 (segment (start 88.265 122.555) (end 99.06 122.555) (width 0.3048) (layer B.Cu) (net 14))
 (segment (start 99.06 122.555) (end 101.22 122.555) (width 0.3048) (layer F.Cu) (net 14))
 (segment (start 103.8075 125.095) (end 101.22 125.095) (width 0.3048) (layer F.Cu) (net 4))
 (segment (start 103.8075 125.095) (end 103.8075 123.19) (width 0.3048) (layer F.Cu) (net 4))
 (segment (start 103.8075 117.475) (end 101.22 117.475) (width 0.3048) (layer F.Cu) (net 7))
 (segment (start 93.0425 106.68) (end 92.4075 106.045) (width 0.3048) (layer F.Cu) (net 24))
 (segment (start 95.09 106.68) (end 93.0425 106.68) (width 0.3048) (layer F.Cu) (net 24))
 (segment (start 92.4075 106.045) (end 92.4075 104.14) (width 0.3048) (layer F.Cu) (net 24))
 (segment (start 100.49 110.49) (end 103.8075 110.49) (width 0.3048) (layer F.Cu) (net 23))
 (segment (start 100.49 107.95) (end 100.49 109.22) (width 0.3048) (layer F.Cu) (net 21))
 (segment (start 93.0425 109.22) (end 95.09 109.22) (width 0.3048) (layer F.Cu) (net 9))
 (segment (start 92.4075 109.855) (end 93.0425 109.22) (width 0.3048) (layer F.Cu) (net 9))
 (segment (start 92.3775 109.855) (end 90.4725 111.76) (width 0.3048) (layer F.Cu) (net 9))
 (segment (start 92.4075 109.855) (end 92.3775 109.855) (width 0.3048) (layer F.Cu) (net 9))
 (segment (start 99.02 93.385) (end 95.25 97.155) (width 1.016) (layer F.Cu) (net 3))
 (segment (start 99.02 93.345) (end 99.02 93.385) (width 1.016) (layer F.Cu) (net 3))
 (segment (start 95.25 95.339) (end 95.161 95.25) (width 1.016) (layer F.Cu) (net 3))
 (segment (start 95.25 97.155) (end 95.25 95.339) (width 1.016) (layer F.Cu) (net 3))
 (segment (start 95.161 95.25) (end 91.86566 95.25) (width 1.016) (layer F.Cu) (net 3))
 (segment (start 91.86566 95.25) (end 90.805 95.25) (width 1.016) (layer F.Cu) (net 3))
 (segment (start 96.52 86.32) (end 100.29 82.55) (width 1.778) (layer F.Cu) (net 6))
 (segment (start 96.52 86.36) (end 96.52 86.32) (width 1.778) (layer F.Cu) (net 6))
 (segment (start 101.6 89.965202) (end 101.6 91.44) (width 1.778) (layer F.Cu) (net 6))
 (segment (start 97.994798 86.36) (end 101.6 89.965202) (width 1.778) (layer F.Cu) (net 6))
 (segment (start 104.2 94.04) (end 106.045 94.04) (width 1.778) (layer F.Cu) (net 6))
 (segment (start 101.6 91.44) (end 104.2 94.04) (width 1.778) (layer F.Cu) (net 6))
 (segment (start 96.52 86.36) (end 97.994798 86.36) (width 1.778) (layer F.Cu) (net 6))
 (segment (start 98.18 114.6698) (end 98.18 113.665) (width 0.3048) (layer F.Cu) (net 26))
 (segment (start 98.18 116.405) (end 98.18 114.6698) (width 0.3048) (layer F.Cu) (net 26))
 (segment (start 100.52 118.745) (end 98.18 116.405) (width 0.3048) (layer F.Cu) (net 26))
 (segment (start 101.22 118.745) (end 100.52 118.745) (width 0.3048) (layer F.Cu) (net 26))
 (segment (start 95.09 107.95) (end 92.4075 107.95) (width 0.3048) (layer F.Cu) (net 25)))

